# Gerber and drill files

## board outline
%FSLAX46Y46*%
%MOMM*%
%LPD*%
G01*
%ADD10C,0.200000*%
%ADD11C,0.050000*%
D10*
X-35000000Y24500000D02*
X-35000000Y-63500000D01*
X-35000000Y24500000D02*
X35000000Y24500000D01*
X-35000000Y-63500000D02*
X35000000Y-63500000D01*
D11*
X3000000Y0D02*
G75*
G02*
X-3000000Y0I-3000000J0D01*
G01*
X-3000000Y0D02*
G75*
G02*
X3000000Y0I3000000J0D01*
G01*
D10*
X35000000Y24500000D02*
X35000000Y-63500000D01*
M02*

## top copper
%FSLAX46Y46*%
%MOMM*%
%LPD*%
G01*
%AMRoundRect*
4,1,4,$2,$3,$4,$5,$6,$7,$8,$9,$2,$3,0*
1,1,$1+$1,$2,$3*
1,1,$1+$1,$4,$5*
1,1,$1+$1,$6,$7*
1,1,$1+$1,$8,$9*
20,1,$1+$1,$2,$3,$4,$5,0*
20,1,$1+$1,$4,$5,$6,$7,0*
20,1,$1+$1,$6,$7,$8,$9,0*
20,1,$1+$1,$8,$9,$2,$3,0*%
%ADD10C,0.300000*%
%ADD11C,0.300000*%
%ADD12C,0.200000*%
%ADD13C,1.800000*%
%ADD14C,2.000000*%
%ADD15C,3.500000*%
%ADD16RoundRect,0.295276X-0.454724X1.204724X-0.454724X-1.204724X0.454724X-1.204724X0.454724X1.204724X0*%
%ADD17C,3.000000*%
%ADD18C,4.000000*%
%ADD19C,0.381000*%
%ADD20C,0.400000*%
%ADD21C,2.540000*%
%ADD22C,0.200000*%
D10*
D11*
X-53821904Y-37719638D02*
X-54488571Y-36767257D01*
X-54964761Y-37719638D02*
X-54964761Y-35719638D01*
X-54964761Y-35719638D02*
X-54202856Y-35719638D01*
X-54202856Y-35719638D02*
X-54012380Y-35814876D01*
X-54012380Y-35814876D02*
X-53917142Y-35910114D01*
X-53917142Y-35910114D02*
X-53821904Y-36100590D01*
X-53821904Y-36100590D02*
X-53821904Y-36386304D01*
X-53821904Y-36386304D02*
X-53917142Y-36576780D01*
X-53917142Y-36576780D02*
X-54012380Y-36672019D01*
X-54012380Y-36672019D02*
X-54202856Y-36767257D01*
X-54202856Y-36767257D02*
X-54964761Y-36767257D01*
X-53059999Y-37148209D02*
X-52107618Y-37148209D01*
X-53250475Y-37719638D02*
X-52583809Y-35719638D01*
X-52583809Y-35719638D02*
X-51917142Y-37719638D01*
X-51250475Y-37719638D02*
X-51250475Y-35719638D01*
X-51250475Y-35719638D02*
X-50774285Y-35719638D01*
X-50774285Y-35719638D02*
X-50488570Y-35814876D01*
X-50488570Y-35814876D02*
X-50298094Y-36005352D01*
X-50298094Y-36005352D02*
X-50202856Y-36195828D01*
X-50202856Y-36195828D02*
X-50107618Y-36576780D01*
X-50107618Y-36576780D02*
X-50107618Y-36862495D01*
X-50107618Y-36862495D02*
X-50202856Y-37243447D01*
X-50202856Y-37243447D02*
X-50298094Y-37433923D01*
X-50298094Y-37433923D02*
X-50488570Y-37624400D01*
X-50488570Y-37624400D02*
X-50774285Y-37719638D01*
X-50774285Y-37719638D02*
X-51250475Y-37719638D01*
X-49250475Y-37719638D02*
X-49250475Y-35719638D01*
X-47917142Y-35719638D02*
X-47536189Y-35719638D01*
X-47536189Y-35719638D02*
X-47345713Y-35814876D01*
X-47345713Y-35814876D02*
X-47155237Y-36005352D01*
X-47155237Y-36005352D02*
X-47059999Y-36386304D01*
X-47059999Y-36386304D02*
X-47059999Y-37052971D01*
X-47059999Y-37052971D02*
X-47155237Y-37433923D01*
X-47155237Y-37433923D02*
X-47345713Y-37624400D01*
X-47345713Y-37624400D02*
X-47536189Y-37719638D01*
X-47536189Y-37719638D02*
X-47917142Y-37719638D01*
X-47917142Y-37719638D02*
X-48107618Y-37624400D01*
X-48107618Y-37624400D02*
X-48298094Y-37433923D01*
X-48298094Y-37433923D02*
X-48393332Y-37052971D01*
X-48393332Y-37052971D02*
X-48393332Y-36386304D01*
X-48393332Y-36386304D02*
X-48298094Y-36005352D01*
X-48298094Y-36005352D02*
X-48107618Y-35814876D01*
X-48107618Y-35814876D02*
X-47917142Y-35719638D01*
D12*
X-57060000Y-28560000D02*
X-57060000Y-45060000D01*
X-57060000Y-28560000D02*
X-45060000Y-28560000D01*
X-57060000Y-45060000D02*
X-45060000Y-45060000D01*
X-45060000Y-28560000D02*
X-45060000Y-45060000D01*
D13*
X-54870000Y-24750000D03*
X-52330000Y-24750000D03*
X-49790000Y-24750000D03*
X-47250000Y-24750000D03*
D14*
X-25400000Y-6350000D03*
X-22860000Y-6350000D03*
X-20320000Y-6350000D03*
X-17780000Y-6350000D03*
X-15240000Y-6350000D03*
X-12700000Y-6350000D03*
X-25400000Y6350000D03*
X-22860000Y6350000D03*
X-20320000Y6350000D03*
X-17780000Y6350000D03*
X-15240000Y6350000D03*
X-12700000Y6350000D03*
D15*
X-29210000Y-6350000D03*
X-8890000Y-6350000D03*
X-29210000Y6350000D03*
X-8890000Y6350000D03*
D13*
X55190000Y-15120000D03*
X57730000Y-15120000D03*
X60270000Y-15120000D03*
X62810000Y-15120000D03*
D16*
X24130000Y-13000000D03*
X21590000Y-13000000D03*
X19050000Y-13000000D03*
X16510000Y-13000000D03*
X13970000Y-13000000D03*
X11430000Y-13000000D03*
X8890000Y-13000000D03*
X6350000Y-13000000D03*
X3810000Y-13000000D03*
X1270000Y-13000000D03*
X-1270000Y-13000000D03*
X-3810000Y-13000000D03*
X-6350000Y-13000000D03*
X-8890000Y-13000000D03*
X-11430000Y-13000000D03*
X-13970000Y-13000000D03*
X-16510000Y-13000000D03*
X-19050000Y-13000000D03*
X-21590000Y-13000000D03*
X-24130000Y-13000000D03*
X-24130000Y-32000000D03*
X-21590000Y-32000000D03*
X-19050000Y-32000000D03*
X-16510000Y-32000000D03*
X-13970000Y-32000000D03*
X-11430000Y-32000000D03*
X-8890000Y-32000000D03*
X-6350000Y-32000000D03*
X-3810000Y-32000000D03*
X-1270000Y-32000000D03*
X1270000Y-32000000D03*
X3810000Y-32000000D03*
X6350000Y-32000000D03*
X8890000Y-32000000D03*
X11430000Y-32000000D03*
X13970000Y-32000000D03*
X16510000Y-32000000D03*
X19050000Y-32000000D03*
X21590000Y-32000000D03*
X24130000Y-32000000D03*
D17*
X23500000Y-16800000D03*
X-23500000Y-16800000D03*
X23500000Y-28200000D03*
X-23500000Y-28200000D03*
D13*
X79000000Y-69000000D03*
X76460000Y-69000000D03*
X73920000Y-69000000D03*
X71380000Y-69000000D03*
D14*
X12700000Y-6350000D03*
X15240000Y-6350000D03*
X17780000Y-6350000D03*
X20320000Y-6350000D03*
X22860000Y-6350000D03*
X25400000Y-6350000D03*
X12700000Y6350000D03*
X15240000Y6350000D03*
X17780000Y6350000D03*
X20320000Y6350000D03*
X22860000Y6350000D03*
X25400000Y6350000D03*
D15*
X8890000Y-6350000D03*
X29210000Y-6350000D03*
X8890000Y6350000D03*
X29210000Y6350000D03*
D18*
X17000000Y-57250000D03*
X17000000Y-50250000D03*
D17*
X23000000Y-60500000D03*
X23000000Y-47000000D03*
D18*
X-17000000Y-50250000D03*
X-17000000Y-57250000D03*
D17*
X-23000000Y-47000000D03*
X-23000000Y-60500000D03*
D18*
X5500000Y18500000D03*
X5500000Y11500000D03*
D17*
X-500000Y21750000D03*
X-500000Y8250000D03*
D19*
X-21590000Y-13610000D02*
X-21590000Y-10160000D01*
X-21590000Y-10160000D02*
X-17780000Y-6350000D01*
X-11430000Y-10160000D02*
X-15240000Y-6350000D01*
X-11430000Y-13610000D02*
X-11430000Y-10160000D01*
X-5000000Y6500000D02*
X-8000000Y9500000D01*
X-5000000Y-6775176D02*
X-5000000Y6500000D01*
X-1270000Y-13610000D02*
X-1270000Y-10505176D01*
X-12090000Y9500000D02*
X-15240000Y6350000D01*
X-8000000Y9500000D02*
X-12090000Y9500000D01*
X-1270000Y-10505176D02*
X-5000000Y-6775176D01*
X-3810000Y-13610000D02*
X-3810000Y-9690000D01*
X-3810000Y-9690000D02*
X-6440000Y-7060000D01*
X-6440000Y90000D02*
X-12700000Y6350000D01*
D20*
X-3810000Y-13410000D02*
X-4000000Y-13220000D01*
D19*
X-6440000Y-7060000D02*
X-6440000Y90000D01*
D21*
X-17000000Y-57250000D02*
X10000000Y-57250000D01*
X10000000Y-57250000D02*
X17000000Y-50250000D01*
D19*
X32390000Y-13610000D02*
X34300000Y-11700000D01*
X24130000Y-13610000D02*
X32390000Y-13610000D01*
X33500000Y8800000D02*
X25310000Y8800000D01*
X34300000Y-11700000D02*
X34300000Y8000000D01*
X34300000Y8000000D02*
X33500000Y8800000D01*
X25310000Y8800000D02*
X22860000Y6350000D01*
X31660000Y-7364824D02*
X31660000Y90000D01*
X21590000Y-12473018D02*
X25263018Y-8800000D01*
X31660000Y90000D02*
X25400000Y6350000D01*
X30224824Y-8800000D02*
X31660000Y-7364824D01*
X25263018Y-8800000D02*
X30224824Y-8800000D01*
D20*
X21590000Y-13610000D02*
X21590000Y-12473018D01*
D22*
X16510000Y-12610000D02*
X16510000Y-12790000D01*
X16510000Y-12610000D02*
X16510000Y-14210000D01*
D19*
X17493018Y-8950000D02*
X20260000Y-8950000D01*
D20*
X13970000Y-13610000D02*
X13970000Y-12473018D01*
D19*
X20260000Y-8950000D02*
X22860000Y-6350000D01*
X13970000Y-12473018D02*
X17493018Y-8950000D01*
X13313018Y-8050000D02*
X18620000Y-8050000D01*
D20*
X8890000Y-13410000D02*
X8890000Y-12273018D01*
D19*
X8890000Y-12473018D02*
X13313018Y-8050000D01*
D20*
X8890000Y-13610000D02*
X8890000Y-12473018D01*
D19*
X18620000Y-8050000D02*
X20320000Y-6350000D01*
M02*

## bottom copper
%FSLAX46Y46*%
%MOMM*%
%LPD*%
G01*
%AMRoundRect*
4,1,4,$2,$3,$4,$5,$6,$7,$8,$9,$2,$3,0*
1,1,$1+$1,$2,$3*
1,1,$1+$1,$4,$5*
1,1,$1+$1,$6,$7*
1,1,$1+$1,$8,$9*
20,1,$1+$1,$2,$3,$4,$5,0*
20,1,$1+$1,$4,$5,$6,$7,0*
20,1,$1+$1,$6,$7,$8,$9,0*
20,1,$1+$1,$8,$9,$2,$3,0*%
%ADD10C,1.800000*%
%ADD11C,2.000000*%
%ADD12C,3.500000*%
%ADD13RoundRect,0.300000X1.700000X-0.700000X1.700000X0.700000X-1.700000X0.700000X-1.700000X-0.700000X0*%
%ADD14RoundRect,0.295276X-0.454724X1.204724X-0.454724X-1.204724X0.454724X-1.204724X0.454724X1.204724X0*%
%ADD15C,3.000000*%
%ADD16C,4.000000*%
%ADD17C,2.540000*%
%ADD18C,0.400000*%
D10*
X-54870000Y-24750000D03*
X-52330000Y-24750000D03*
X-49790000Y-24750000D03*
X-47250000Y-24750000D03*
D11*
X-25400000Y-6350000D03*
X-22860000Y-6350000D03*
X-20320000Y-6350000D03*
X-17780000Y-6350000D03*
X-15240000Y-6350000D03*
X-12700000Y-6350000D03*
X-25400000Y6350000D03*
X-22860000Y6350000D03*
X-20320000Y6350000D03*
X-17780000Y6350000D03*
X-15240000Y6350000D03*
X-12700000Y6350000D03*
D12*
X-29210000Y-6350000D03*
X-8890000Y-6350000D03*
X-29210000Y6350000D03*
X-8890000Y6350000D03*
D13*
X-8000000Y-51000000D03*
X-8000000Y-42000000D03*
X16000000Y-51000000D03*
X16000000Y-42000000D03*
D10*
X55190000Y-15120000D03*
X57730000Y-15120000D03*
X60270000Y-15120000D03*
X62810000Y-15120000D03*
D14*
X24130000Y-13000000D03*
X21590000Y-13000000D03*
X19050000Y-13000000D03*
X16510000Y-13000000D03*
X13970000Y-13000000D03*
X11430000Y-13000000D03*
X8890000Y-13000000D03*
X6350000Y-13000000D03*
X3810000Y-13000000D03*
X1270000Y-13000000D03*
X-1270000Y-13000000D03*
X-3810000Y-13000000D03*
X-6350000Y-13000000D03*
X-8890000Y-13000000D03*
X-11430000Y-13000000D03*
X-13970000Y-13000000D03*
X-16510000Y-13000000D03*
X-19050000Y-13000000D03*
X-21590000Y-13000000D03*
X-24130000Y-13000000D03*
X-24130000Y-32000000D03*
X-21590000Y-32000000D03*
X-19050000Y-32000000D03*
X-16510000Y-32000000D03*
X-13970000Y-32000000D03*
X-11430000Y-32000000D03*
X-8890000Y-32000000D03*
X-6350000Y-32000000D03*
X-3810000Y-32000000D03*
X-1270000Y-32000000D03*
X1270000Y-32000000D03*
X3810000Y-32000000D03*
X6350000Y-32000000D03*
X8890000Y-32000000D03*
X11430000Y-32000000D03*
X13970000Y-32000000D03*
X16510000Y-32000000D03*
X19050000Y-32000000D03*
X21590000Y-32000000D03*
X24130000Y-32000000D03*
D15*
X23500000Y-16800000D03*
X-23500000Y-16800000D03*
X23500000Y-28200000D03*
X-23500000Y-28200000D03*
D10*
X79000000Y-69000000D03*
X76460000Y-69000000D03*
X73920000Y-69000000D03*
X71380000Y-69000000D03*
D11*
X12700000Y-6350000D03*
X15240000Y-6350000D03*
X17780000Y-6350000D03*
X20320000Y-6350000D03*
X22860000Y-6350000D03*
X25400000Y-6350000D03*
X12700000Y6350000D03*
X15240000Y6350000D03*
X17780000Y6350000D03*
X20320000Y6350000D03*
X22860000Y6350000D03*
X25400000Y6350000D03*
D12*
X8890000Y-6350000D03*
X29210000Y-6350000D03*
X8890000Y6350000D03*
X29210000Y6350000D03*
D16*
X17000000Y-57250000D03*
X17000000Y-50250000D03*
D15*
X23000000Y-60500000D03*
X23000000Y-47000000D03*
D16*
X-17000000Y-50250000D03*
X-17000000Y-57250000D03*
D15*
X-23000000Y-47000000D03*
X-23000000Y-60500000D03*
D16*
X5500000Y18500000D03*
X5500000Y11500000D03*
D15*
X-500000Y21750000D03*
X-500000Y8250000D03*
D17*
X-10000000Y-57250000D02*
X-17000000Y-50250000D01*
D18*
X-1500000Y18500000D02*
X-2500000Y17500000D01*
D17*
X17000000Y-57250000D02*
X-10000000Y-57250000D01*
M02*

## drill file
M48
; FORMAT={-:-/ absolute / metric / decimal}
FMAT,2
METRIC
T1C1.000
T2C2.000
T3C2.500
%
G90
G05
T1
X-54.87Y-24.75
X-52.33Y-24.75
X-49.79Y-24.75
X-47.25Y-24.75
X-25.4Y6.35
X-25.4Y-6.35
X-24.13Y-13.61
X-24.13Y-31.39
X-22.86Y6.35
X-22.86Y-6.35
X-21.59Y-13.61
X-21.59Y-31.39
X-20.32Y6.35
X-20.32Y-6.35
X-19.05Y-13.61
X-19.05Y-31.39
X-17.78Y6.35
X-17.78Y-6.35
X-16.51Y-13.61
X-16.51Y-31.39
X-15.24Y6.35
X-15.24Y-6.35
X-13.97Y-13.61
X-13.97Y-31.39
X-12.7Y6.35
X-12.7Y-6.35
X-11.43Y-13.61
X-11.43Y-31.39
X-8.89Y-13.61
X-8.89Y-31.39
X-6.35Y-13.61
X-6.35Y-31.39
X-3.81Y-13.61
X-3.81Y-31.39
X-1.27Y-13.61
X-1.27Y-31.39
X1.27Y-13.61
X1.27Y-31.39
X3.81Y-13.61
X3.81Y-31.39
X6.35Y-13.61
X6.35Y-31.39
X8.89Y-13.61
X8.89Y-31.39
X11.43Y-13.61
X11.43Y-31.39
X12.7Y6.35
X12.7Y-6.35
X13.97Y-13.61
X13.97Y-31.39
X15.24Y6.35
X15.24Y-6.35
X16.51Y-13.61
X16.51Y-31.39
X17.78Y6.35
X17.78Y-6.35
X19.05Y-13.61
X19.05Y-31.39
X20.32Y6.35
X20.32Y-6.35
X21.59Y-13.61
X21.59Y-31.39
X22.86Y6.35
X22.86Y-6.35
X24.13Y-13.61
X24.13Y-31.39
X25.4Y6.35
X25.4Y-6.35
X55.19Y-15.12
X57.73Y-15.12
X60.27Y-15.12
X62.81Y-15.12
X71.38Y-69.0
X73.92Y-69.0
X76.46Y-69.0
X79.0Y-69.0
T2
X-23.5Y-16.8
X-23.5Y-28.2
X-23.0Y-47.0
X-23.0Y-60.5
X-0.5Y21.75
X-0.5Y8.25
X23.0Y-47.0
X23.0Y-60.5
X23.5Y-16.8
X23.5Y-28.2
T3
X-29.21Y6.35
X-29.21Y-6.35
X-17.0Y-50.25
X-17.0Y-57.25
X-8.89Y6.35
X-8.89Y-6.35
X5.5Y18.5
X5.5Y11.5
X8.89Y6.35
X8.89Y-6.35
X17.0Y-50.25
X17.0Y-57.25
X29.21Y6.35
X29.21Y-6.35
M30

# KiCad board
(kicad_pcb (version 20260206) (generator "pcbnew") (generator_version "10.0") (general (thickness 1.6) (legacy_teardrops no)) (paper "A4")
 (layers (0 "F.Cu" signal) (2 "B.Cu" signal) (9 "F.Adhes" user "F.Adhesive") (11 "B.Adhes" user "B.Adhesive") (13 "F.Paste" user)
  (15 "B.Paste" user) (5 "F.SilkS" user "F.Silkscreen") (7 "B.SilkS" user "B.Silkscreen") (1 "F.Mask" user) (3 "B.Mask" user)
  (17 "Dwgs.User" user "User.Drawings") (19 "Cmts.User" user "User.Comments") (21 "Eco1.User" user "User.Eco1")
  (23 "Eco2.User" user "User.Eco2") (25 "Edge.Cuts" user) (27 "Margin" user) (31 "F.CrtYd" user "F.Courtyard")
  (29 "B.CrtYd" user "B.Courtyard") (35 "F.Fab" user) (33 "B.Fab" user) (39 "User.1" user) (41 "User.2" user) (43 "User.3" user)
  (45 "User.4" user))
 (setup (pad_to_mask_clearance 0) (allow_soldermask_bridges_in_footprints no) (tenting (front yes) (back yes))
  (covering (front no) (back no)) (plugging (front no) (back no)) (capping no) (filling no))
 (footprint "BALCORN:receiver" (layer "F.Cu") (at -51.06 36.81)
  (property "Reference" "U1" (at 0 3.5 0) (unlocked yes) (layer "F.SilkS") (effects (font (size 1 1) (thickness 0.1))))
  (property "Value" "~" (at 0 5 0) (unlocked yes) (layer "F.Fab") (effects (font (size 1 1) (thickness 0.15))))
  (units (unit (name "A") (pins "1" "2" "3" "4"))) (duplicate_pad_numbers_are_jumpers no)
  (fp_line (start -6 -8.25) (end -6 8.25) (stroke (width 0.2) (type default)) (layer "F.Cu"))
  (fp_line (start -6 -8.25) (end 6 -8.25) (stroke (width 0.2) (type default)) (layer "F.Cu"))
  (fp_line (start -6 8.25) (end 6 8.25) (stroke (width 0.2) (type default)) (layer "F.Cu"))
  (fp_line (start 6 -8.25) (end 6 8.25) (stroke (width 0.2) (type default)) (layer "F.Cu"))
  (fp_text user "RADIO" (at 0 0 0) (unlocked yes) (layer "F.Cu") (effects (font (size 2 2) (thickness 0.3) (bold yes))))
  (pad "1" thru_hole circle (at -3.81 -12.06) (size 1.8 1.8) (drill 1) (layers "*.Cu" "*.Mask") (remove_unused_layers no)
   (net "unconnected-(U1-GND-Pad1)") (thermal_bridge_angle 90))
  (pad "2" thru_hole circle (at -1.27 -12.06) (size 1.8 1.8) (drill 1) (layers "*.Cu" "*.Mask") (remove_unused_layers no)
   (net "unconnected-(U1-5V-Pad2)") (thermal_bridge_angle 90))
  (pad "3" thru_hole circle (at 1.27 -12.06) (size 1.8 1.8) (drill 1) (layers "*.Cu" "*.Mask") (remove_unused_layers no)
   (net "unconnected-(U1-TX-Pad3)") (thermal_bridge_angle 90))
  (pad "4" thru_hole circle (at 3.81 -12.06) (size 1.8 1.8) (drill 1) (layers "*.Cu" "*.Mask") (remove_unused_layers no)
   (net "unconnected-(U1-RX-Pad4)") (thermal_bridge_angle 90)))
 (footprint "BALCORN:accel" (layer "F.Cu") (at -19.05 0 90)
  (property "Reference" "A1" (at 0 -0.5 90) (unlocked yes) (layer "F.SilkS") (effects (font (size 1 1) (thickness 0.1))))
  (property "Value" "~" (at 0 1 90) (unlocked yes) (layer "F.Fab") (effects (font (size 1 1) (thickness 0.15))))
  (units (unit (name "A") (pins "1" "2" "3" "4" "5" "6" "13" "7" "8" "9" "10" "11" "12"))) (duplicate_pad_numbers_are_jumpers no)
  (pad "1" thru_hole circle (at -6.35 -6.35 90) (size 2 2) (drill 1) (layers "*.Cu" "*.Mask") (remove_unused_layers no) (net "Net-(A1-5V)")
   (thermal_bridge_angle 90))
  (pad "2" thru_hole circle (at -6.35 -3.81 90) (size 2 2) (drill 1) (layers "*.Cu" "*.Mask") (remove_unused_layers no)
   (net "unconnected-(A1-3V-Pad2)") (thermal_bridge_angle 90))
  (pad "3" thru_hole circle (at -6.35 -1.27 90) (size 2 2) (drill 1) (layers "*.Cu" "*.Mask") (remove_unused_layers no)
   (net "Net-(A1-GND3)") (thermal_bridge_angle 90))
  (pad "4" thru_hole circle (at -6.35 1.27 90) (size 2 2) (drill 1) (layers "*.Cu" "*.Mask") (remove_unused_layers no) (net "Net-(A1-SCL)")
   (thermal_bridge_angle 90))
  (pad "5" thru_hole circle (at -6.35 3.81 90) (size 2 2) (drill 1) (layers "*.Cu" "*.Mask") (remove_unused_layers no) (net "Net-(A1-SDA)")
   (thermal_bridge_angle 90))
  (pad "6" thru_hole circle (at -6.35 6.35 90) (size 2 2) (drill 1) (layers "*.Cu" "*.Mask") (remove_unused_layers no)
   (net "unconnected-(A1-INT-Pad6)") (thermal_bridge_angle 90))
  (pad "7" thru_hole circle (at 6.35 -6.35 90) (size 2 2) (drill 1) (layers "*.Cu" "*.Mask") (remove_unused_layers no)
   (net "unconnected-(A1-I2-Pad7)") (thermal_bridge_angle 90))
  (pad "8" thru_hole circle (at 6.35 -3.81 90) (size 2 2) (drill 1) (layers "*.Cu" "*.Mask") (remove_unused_layers no)
   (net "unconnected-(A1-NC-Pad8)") (thermal_bridge_angle 90))
  (pad "9" thru_hole circle (at 6.35 -1.27 90) (size 2 2) (drill 1) (layers "*.Cu" "*.Mask") (remove_unused_layers no)
   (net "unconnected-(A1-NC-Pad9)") (thermal_bridge_angle 90))
  (pad "10" thru_hole circle (at 6.35 1.27 90) (size 2 2) (drill 1) (layers "*.Cu" "*.Mask") (remove_unused_layers no)
   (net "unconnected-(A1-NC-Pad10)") (thermal_bridge_angle 90))
  (pad "11" thru_hole circle (at 6.35 3.81 90) (size 2 2) (drill 1) (layers "*.Cu" "*.Mask") (remove_unused_layers no) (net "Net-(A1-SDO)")
   (thermal_bridge_angle 90))
  (pad "12" thru_hole circle (at 6.35 6.35 90) (size 2 2) (drill 1) (layers "*.Cu" "*.Mask") (remove_unused_layers no) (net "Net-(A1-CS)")
   (thermal_bridge_angle 90))
  (pad "13" thru_hole circle (at -6.35 -10.16 90) (size 3.5 3.5) (drill 2.5) (layers "*.Cu" "*.Mask") (remove_unused_layers no)
   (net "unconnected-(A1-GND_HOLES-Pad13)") (thermal_bridge_angle 90))
  (pad "13" thru_hole circle (at -6.35 10.16 90) (size 3.5 3.5) (drill 2.5) (layers "*.Cu" "*.Mask") (remove_unused_layers no)
   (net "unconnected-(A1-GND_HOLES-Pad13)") (thermal_bridge_angle 90))
  (pad "13" thru_hole circle (at 6.35 -10.16 90) (size 3.5 3.5) (drill 2.5) (layers "*.Cu" "*.Mask") (remove_unused_layers no)
   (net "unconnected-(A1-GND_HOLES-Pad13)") (thermal_bridge_angle 90))
  (pad "13" thru_hole circle (at 6.35 10.16 90) (size 3.5 3.5) (drill 2.5) (layers "*.Cu" "*.Mask") (remove_unused_layers no)
   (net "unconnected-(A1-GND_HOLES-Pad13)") (thermal_bridge_angle 90)))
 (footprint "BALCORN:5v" (layer "F.Cu") (at 4 46.5 90)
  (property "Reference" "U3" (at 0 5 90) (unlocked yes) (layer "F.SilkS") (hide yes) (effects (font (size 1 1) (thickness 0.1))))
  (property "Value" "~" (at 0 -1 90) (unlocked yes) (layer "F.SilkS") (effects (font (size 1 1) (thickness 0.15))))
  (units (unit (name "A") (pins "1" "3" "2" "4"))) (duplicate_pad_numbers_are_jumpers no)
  (pad "1" smd roundrect (at -4.5 -12 90) (size 2 4) (layers "*.Mask" "B.Cu") (roundrect_rratio 0.15) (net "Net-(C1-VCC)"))
  (pad "2" smd roundrect (at 4.5 -12 90) (size 2 4) (layers "*.Mask" "B.Cu") (roundrect_rratio 0.15) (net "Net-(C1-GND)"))
  (pad "3" smd roundrect (at -4.5 12 90) (size 2 4) (layers "*.Mask" "B.Cu") (roundrect_rratio 0.15) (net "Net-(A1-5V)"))
  (pad "4" smd roundrect (at 4.5 12 90) (size 2 4) (layers "*.Mask" "B.Cu") (roundrect_rratio 0.15) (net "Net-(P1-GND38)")))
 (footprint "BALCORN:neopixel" (layer "F.Cu") (at 59 15.12)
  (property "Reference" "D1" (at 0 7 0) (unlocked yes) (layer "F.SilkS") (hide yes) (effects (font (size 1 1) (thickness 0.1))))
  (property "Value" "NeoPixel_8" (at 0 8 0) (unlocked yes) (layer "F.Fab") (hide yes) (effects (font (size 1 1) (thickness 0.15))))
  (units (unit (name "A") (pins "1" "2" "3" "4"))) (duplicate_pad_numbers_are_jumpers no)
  (pad "1" thru_hole circle (at -3.81 0) (size 1.8 1.8) (drill 1) (layers "*.Cu" "*.Mask") (remove_unused_layers no)
   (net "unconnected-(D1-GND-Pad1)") (thermal_bridge_angle 90))
  (pad "2" thru_hole circle (at -1.27 0) (size 1.8 1.8) (drill 1) (layers "*.Cu" "*.Mask") (remove_unused_layers no)
   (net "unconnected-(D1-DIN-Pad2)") (thermal_bridge_angle 90))
  (pad "3" thru_hole circle (at 1.27 0) (size 1.8 1.8) (drill 1) (layers "*.Cu" "*.Mask") (remove_unused_layers no)
   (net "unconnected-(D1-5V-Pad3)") (thermal_bridge_angle 90))
  (pad "4" thru_hole circle (at 3.81 0) (size 1.8 1.8) (drill 1) (layers "*.Cu" "*.Mask") (remove_unused_layers no)
   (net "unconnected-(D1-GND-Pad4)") (thermal_bridge_angle 90)))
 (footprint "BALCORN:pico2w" (layer "F.Cu") (at 0 22.5 -90)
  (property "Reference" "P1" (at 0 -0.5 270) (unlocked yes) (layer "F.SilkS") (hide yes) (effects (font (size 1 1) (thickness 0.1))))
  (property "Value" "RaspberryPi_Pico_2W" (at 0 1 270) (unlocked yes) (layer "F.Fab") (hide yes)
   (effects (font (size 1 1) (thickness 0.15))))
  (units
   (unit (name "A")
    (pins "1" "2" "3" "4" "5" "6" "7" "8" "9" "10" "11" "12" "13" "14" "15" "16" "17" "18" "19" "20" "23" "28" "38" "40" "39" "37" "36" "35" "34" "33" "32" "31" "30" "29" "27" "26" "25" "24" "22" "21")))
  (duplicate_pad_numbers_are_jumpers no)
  (pad "1" thru_hole roundrect (at -8.89 -24.13 270) (size 3 1.5) (drill 1 (offset -0.61 0)) (layers "*.Cu" "*.Mask")
   (remove_unused_layers no) (roundrect_rratio 0.1968503937) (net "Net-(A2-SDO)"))
  (pad "2" thru_hole roundrect (at -8.89 -21.59 270) (size 3 1.5) (drill 1 (offset -0.61 0)) (layers "*.Cu" "*.Mask")
   (remove_unused_layers no) (roundrect_rratio 0.1968503937) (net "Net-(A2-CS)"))
  (pad "3" thru_hole roundrect (at -8.89 -19.05 270) (size 3 1.5) (drill 1 (offset -0.61 0)) (layers "*.Cu" "*.Mask")
   (remove_unused_layers no) (roundrect_rratio 0.1968503937) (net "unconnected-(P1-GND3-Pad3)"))
  (pad "4" thru_hole roundrect (at -8.89 -16.51 270) (size 3 1.5) (drill 1 (offset -0.61 0)) (layers "*.Cu" "*.Mask")
   (remove_unused_layers no) (roundrect_rratio 0.1968503937) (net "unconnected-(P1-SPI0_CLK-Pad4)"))
  (pad "5" thru_hole roundrect (at -8.89 -13.97 270) (size 3 1.5) (drill 1 (offset -0.61 0)) (layers "*.Cu" "*.Mask")
   (remove_unused_layers no) (roundrect_rratio 0.1968503937) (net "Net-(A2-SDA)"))
  (pad "6" thru_hole roundrect (at -8.89 -11.43 270) (size 3 1.5) (drill 1 (offset -0.61 0)) (layers "*.Cu" "*.Mask")
   (remove_unused_layers no) (roundrect_rratio 0.1968503937) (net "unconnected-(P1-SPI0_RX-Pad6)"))
  (pad "7" thru_hole roundrect (at -8.89 -8.89 270) (size 3 1.5) (drill 1 (offset -0.61 0)) (layers "*.Cu" "*.Mask")
   (remove_unused_layers no) (roundrect_rratio 0.1968503937) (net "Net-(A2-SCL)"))
  (pad "8" thru_hole roundrect (at -8.89 -6.35 270) (size 3 1.5) (drill 1 (offset -0.61 0)) (layers "*.Cu" "*.Mask")
   (remove_unused_layers no) (roundrect_rratio 0.1968503937) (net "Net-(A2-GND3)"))
  (pad "9" thru_hole roundrect (at -8.89 -3.81 270) (size 3 1.5) (drill 1 (offset -0.61 0)) (layers "*.Cu" "*.Mask")
   (remove_unused_layers no) (roundrect_rratio 0.1968503937) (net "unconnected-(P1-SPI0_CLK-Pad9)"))
  (pad "10" thru_hole roundrect (at -8.89 -1.27 270) (size 3 1.5) (drill 1 (offset -0.61 0)) (layers "*.Cu" "*.Mask")
   (remove_unused_layers no) (roundrect_rratio 0.1968503937) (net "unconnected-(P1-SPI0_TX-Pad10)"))
  (pad "11" thru_hole roundrect (at -8.89 1.27 270) (size 3 1.5) (drill 1 (offset -0.61 0)) (layers "*.Cu" "*.Mask")
   (remove_unused_layers no) (roundrect_rratio 0.1968503937) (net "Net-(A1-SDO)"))
  (pad "12" thru_hole roundrect (at -8.89 3.81 270) (size 3 1.5) (drill 1 (offset -0.61 0)) (layers "*.Cu" "*.Mask")
   (remove_unused_layers no) (roundrect_rratio 0.1968503937) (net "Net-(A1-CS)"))
  (pad "13" thru_hole roundrect (at -8.89 6.35 270) (size 3 1.5) (drill 1 (offset -0.61 0)) (layers "*.Cu" "*.Mask")
   (remove_unused_layers no) (roundrect_rratio 0.1968503937) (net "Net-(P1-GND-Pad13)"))
  (pad "14" thru_hole roundrect (at -8.89 8.89 270) (size 3 1.5) (drill 1 (offset -0.61 0)) (layers "*.Cu" "*.Mask")
   (remove_unused_layers no) (roundrect_rratio 0.1968503937) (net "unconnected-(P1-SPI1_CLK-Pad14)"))
  (pad "15" thru_hole roundrect (at -8.89 11.43 270) (size 3 1.5) (drill 1 (offset -0.61 0)) (layers "*.Cu" "*.Mask")
   (remove_unused_layers no) (roundrect_rratio 0.1968503937) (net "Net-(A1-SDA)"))
  (pad "16" thru_hole roundrect (at -8.89 13.97 270) (size 3 1.5) (drill 1 (offset -0.61 0)) (layers "*.Cu" "*.Mask")
   (remove_unused_layers no) (roundrect_rratio 0.1968503937) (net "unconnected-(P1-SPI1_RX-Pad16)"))
  (pad "17" thru_hole roundrect (at -8.89 16.51 270) (size 3 1.5) (drill 1 (offset -0.61 0)) (layers "*.Cu" "*.Mask")
   (remove_unused_layers no) (roundrect_rratio 0.1968503937) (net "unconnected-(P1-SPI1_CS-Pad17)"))
  (pad "18" thru_hole roundrect (at -8.89 19.05 270) (size 3 1.5) (drill 1 (offset -0.61 0)) (layers "*.Cu" "*.Mask")
   (remove_unused_layers no) (roundrect_rratio 0.1968503937) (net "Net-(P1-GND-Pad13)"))
  (pad "19" thru_hole roundrect (at -8.89 21.59 270) (size 3 1.5) (drill 1 (offset -0.61 0)) (layers "*.Cu" "*.Mask")
   (remove_unused_layers no) (roundrect_rratio 0.1968503937) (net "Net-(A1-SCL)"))
  (pad "20" thru_hole roundrect (at -8.89 24.13 270) (size 3 1.5) (drill 1 (offset -0.61 0)) (layers "*.Cu" "*.Mask")
   (remove_unused_layers no) (roundrect_rratio 0.1968503937) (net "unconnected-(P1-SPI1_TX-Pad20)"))
  (pad "21" thru_hole roundrect (at 8.89 24.13 270) (size 3 1.5) (drill 1 (offset 0.61 0)) (layers "*.Cu" "*.Mask")
   (remove_unused_layers no) (roundrect_rratio 0.1968503937) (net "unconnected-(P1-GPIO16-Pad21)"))
  (pad "22" thru_hole roundrect (at 8.89 21.59 270) (size 3 1.5) (drill 1 (offset 0.61 0)) (layers "*.Cu" "*.Mask")
   (remove_unused_layers no) (roundrect_rratio 0.1968503937) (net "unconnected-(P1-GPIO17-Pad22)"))
  (pad "23" thru_hole roundrect (at 8.89 19.05 270) (size 3 1.5) (drill 1 (offset 0.61 0)) (layers "*.Cu" "*.Mask")
   (remove_unused_layers no) (roundrect_rratio 0.1968503937) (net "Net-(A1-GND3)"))
  (pad "24" thru_hole roundrect (at 8.89 16.51 270) (size 3 1.5) (drill 1 (offset 0.61 0)) (layers "*.Cu" "*.Mask")
   (remove_unused_layers no) (roundrect_rratio 0.1968503937) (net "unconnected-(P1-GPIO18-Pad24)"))
  (pad "25" thru_hole roundrect (at 8.89 13.97 270) (size 3 1.5) (drill 1 (offset 0.61 0)) (layers "*.Cu" "*.Mask")
   (remove_unused_layers no) (roundrect_rratio 0.1968503937) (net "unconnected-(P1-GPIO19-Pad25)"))
  (pad "26" thru_hole roundrect (at 8.89 11.43 270) (size 3 1.5) (drill 1 (offset 0.61 0)) (layers "*.Cu" "*.Mask")
   (remove_unused_layers no) (roundrect_rratio 0.1968503937) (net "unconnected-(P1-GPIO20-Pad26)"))
  (pad "27" thru_hole roundrect (at 8.89 8.89 270) (size 3 1.5) (drill 1 (offset 0.61 0)) (layers "*.Cu" "*.Mask") (remove_unused_layers no)
   (roundrect_rratio 0.1968503937) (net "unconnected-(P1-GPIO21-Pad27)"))
  (pad "28" thru_hole roundrect (at 8.89 6.35 270) (size 3 1.5) (drill 1 (offset 0.61 0)) (layers "*.Cu" "*.Mask") (remove_unused_layers no)
   (roundrect_rratio 0.1968503937) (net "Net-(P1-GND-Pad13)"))
  (pad "29" thru_hole roundrect (at 8.89 3.81 270) (size 3 1.5) (drill 1 (offset 0.61 0)) (layers "*.Cu" "*.Mask") (remove_unused_layers no)
   (roundrect_rratio 0.1968503937) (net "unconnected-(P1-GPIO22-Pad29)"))
  (pad "30" thru_hole roundrect (at 8.89 1.27 270) (size 3 1.5) (drill 1 (offset 0.61 0)) (layers "*.Cu" "*.Mask") (remove_unused_layers no)
   (roundrect_rratio 0.1968503937) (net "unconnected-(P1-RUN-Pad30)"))
  (pad "31" thru_hole roundrect (at 8.89 -1.27 270) (size 3 1.5) (drill 1 (offset 0.61 0)) (layers "*.Cu" "*.Mask")
   (remove_unused_layers no) (roundrect_rratio 0.1968503937) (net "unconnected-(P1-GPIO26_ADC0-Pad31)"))
  (pad "32" thru_hole roundrect (at 8.89 -3.81 270) (size 3 1.5) (drill 1 (offset 0.61 0)) (layers "*.Cu" "*.Mask")
   (remove_unused_layers no) (roundrect_rratio 0.1968503937) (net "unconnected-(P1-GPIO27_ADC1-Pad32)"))
  (pad "33" thru_hole roundrect (at 8.89 -6.35 270) (size 3 1.5) (drill 1 (offset 0.61 0)) (layers "*.Cu" "*.Mask")
   (remove_unused_layers no) (roundrect_rratio 0.1968503937) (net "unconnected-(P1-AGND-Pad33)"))
  (pad "34" thru_hole roundrect (at 8.89 -8.89 270) (size 3 1.5) (drill 1 (offset 0.61 0)) (layers "*.Cu" "*.Mask")
   (remove_unused_layers no) (roundrect_rratio 0.1968503937) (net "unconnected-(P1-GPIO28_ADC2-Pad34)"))
  (pad "35" thru_hole roundrect (at 8.89 -11.43 270) (size 3 1.5) (drill 1 (offset 0.61 0)) (layers "*.Cu" "*.Mask")
   (remove_unused_layers no) (roundrect_rratio 0.1968503937) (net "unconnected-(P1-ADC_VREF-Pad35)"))
  (pad "36" thru_hole roundrect (at 8.89 -13.97 270) (size 3 1.5) (drill 1 (offset 0.61 0)) (layers "*.Cu" "*.Mask")
   (remove_unused_layers no) (roundrect_rratio 0.1968503937) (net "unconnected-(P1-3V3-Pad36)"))
  (pad "37" thru_hole roundrect (at 8.89 -16.51 270) (size 3 1.5) (drill 1 (offset 0.61 0)) (layers "*.Cu" "*.Mask")
   (remove_unused_layers no) (roundrect_rratio 0.1968503937) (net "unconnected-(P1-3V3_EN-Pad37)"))
  (pad "38" thru_hole roundrect (at 8.89 -19.05 270) (size 3 1.5) (drill 1 (offset 0.61 0)) (layers "*.Cu" "*.Mask")
   (remove_unused_layers no) (roundrect_rratio 0.1968503937) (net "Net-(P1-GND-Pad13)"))
  (pad "39" thru_hole roundrect (at 8.89 -21.59 270) (size 3 1.5) (drill 1 (offset 0.61 0)) (layers "*.Cu" "*.Mask")
   (remove_unused_layers no) (roundrect_rratio 0.1968503937) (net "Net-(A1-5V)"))
  (pad "40" thru_hole roundrect (at 8.89 -24.13 270) (size 3 1.5) (drill 1 (offset 0.61 0)) (layers "*.Cu" "*.Mask")
   (remove_unused_layers no) (roundrect_rratio 0.1968503937) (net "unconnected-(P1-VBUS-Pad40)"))
  (pad "41" thru_hole circle (at -5.7 -23.5 270) (size 3 3) (drill 2) (layers "*.Cu" "*.Mask") (remove_unused_layers no)
   (thermal_bridge_angle 90))
  (pad "41" thru_hole circle (at -5.7 23.5 270) (size 3 3) (drill 2) (layers "*.Cu" "*.Mask") (remove_unused_layers no)
   (thermal_bridge_angle 90))
  (pad "41" thru_hole circle (at 5.7 -23.5 270) (size 3 3) (drill 2) (layers "*.Cu" "*.Mask") (remove_unused_layers no)
   (thermal_bridge_angle 90))
  (pad "41" thru_hole circle (at 5.7 23.5 270) (size 3 3) (drill 2) (layers "*.Cu" "*.Mask") (remove_unused_layers no)
   (thermal_bridge_angle 90)))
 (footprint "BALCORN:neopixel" (layer "F.Cu") (at 75.19 69 180)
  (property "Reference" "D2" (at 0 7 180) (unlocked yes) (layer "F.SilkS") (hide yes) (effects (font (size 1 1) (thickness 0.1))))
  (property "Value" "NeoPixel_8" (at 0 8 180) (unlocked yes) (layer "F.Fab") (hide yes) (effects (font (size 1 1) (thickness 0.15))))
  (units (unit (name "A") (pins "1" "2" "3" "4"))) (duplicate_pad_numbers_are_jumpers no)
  (pad "1" thru_hole circle (at -3.81 0 180) (size 1.8 1.8) (drill 1) (layers "*.Cu" "*.Mask") (remove_unused_layers no)
   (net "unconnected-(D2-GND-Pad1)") (thermal_bridge_angle 90))
  (pad "2" thru_hole circle (at -1.27 0 180) (size 1.8 1.8) (drill 1) (layers "*.Cu" "*.Mask") (remove_unused_layers no)
   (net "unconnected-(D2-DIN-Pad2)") (thermal_bridge_angle 90))
  (pad "3" thru_hole circle (at 1.27 0 180) (size 1.8 1.8) (drill 1) (layers "*.Cu" "*.Mask") (remove_unused_layers no)
   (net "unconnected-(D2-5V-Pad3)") (thermal_bridge_angle 90))
  (pad "4" thru_hole circle (at 3.81 0 180) (size 1.8 1.8) (drill 1) (layers "*.Cu" "*.Mask") (remove_unused_layers no)
   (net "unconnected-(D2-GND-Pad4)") (thermal_bridge_angle 90)))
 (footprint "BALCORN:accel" (layer "F.Cu") (at 19.05 0 90)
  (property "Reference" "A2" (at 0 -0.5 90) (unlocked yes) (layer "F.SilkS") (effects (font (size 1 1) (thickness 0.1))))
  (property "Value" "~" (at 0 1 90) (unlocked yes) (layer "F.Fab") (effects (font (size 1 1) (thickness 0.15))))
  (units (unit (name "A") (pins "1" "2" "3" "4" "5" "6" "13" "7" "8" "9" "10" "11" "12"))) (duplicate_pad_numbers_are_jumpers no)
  (pad "1" thru_hole circle (at -6.35 -6.35 90) (size 2 2) (drill 1) (layers "*.Cu" "*.Mask") (remove_unused_layers no)
   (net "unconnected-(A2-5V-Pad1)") (thermal_bridge_angle 90))
  (pad "2" thru_hole circle (at -6.35 -3.81 90) (size 2 2) (drill 1) (layers "*.Cu" "*.Mask") (remove_unused_layers no)
   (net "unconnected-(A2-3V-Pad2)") (thermal_bridge_angle 90))
  (pad "3" thru_hole circle (at -6.35 -1.27 90) (size 2 2) (drill 1) (layers "*.Cu" "*.Mask") (remove_unused_layers no)
   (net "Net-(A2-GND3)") (thermal_bridge_angle 90))
  (pad "4" thru_hole circle (at -6.35 1.27 90) (size 2 2) (drill 1) (layers "*.Cu" "*.Mask") (remove_unused_layers no) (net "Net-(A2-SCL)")
   (thermal_bridge_angle 90))
  (pad "5" thru_hole circle (at -6.35 3.81 90) (size 2 2) (drill 1) (layers "*.Cu" "*.Mask") (remove_unused_layers no) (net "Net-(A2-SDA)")
   (thermal_bridge_angle 90))
  (pad "6" thru_hole circle (at -6.35 6.35 90) (size 2 2) (drill 1) (layers "*.Cu" "*.Mask") (remove_unused_layers no)
   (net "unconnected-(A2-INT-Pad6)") (thermal_bridge_angle 90))
  (pad "7" thru_hole circle (at 6.35 -6.35 90) (size 2 2) (drill 1) (layers "*.Cu" "*.Mask") (remove_unused_layers no)
   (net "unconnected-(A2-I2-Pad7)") (thermal_bridge_angle 90))
  (pad "8" thru_hole circle (at 6.35 -3.81 90) (size 2 2) (drill 1) (layers "*.Cu" "*.Mask") (remove_unused_layers no)
   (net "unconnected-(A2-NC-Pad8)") (thermal_bridge_angle 90))
  (pad "9" thru_hole circle (at 6.35 -1.27 90) (size 2 2) (drill 1) (layers "*.Cu" "*.Mask") (remove_unused_layers no)
   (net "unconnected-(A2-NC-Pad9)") (thermal_bridge_angle 90))
  (pad "10" thru_hole circle (at 6.35 1.27 90) (size 2 2) (drill 1) (layers "*.Cu" "*.Mask") (remove_unused_layers no)
   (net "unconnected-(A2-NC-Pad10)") (thermal_bridge_angle 90))
  (pad "11" thru_hole circle (at 6.35 3.81 90) (size 2 2) (drill 1) (layers "*.Cu" "*.Mask") (remove_unused_layers no) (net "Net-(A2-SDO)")
   (thermal_bridge_angle 90))
  (pad "12" thru_hole circle (at 6.35 6.35 90) (size 2 2) (drill 1) (layers "*.Cu" "*.Mask") (remove_unused_layers no) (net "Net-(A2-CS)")
   (thermal_bridge_angle 90))
  (pad "13" thru_hole circle (at -6.35 -10.16 90) (size 3.5 3.5) (drill 2.5) (layers "*.Cu" "*.Mask") (remove_unused_layers no)
   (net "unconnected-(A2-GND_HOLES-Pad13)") (thermal_bridge_angle 90))
  (pad "13" thru_hole circle (at -6.35 10.16 90) (size 3.5 3.5) (drill 2.5) (layers "*.Cu" "*.Mask") (remove_unused_layers no)
   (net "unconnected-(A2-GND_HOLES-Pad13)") (thermal_bridge_angle 90))
  (pad "13" thru_hole circle (at 6.35 -10.16 90) (size 3.5 3.5) (drill 2.5) (layers "*.Cu" "*.Mask") (remove_unused_layers no)
   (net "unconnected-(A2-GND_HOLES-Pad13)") (thermal_bridge_angle 90))
  (pad "13" thru_hole circle (at 6.35 10.16 90) (size 3.5 3.5) (drill 2.5) (layers "*.Cu" "*.Mask") (remove_unused_layers no)
   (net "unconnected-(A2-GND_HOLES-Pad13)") (thermal_bridge_angle 90)))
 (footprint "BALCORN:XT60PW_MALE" (layer "B.Cu") (at 24.175 53.75 90)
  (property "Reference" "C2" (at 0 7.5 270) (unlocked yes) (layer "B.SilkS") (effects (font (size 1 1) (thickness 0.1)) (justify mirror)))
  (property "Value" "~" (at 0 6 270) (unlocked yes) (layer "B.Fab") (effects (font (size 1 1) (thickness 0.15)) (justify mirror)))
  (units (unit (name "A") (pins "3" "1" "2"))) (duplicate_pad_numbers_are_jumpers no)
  (pad "1" thru_hole circle (at -3.5 -7.175 90) (size 4 4) (drill 2.5) (layers "*.Cu" "*.Mask") (remove_unused_layers no)
   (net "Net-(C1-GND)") (thermal_bridge_angle 90))
  (pad "2" thru_hole circle (at 3.5 -7.175 90) (size 4 4) (drill 2.5) (layers "*.Cu" "*.Mask") (remove_unused_layers no)
   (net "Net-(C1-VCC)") (thermal_bridge_angle 90))
  (pad "3" thru_hole circle (at -6.75 -1.175 90) (size 3 3) (drill 2) (layers "*.Cu" "*.Mask") (remove_unused_layers no)
   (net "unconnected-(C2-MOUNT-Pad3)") (thermal_bridge_angle 90))
  (pad "4" thru_hole circle (at 6.75 -1.175 90) (size 3 3) (drill 2) (layers "*.Cu" "*.Mask") (remove_unused_layers no)
   (thermal_bridge_angle 90)))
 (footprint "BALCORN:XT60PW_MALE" (layer "B.Cu") (at -24.175 53.75 -90)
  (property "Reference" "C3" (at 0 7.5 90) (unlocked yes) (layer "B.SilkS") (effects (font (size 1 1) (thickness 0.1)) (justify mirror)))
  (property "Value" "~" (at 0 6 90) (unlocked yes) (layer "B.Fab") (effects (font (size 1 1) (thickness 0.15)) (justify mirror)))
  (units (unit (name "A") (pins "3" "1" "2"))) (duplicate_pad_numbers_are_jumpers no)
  (pad "1" thru_hole circle (at -3.5 -7.175 270) (size 4 4) (drill 2.5) (layers "*.Cu" "*.Mask") (remove_unused_layers no)
   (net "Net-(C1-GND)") (thermal_bridge_angle 90))
  (pad "2" thru_hole circle (at 3.5 -7.175 270) (size 4 4) (drill 2.5) (layers "*.Cu" "*.Mask") (remove_unused_layers no)
   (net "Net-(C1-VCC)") (thermal_bridge_angle 90))
  (pad "3" thru_hole circle (at -6.75 -1.175 270) (size 3 3) (drill 2) (layers "*.Cu" "*.Mask") (remove_unused_layers no)
   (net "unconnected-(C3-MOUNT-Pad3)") (thermal_bridge_angle 90))
  (pad "4" thru_hole circle (at 6.75 -1.175 270) (size 3 3) (drill 2) (layers "*.Cu" "*.Mask") (remove_unused_layers no)
   (thermal_bridge_angle 90)))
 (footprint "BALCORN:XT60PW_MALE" (layer "B.Cu") (at -1.675 -15 -90)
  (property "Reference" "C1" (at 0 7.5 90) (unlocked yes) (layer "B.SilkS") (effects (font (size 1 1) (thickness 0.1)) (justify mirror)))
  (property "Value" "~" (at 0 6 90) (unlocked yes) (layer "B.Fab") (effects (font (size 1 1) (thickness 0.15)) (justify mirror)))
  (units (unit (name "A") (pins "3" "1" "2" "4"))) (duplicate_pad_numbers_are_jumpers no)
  (pad "1" thru_hole circle (at -3.5 -7.175 270) (size 4 4) (drill 2.5) (layers "*.Cu" "*.Mask") (remove_unused_layers no)
   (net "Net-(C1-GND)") (thermal_bridge_angle 90))
  (pad "2" thru_hole circle (at 3.5 -7.175 270) (size 4 4) (drill 2.5) (layers "*.Cu" "*.Mask") (remove_unused_layers no)
   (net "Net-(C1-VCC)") (thermal_bridge_angle 90))
  (pad "3" thru_hole circle (at -6.75 -1.175 270) (size 3 3) (drill 2) (layers "*.Cu" "*.Mask") (remove_unused_layers no)
   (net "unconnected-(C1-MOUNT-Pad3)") (thermal_bridge_angle 90))
  (pad "4" thru_hole circle (at 6.75 -1.175 270) (size 3 3) (drill 2) (layers "*.Cu" "*.Mask") (remove_unused_layers no)
   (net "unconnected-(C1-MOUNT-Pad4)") (thermal_bridge_angle 90)))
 (gr_line (start -35 -24.5) (end -35 63.5) (stroke (width 0.2) (type default)) (layer "Edge.Cuts"))
 (gr_line (start -35 -24.5) (end 35 -24.5) (stroke (width 0.2) (type default)) (layer "Edge.Cuts"))
 (gr_line (start -35 63.5) (end 35 63.5) (stroke (width 0.2) (type default)) (layer "Edge.Cuts"))
 (gr_circle (center 0 0) (end 3 0) (stroke (width 0.05) (type default)) (fill no) (layer "Edge.Cuts"))
 (gr_line (start 35 -24.5) (end 35 63.5) (stroke (width 0.2) (type default)) (layer "Edge.Cuts"))
 (segment (start -21.59 13.61) (end -21.59 10.16) (width 0.381) (layer "F.Cu") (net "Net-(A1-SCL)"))
 (segment (start -21.59 10.16) (end -17.78 6.35) (width 0.381) (layer "F.Cu") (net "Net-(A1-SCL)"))
 (segment (start -11.43 10.16) (end -15.24 6.35) (width 0.381) (layer "F.Cu") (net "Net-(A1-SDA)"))
 (segment (start -11.43 13.61) (end -11.43 10.16) (width 0.381) (layer "F.Cu") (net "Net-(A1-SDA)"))
 (segment (start -5 -6.5) (end -8 -9.5) (width 0.381) (layer "F.Cu") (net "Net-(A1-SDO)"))
 (segment (start -5 6.775176) (end -5 -6.5) (width 0.381) (layer "F.Cu") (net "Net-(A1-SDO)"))
 (segment (start -1.27 13.61) (end -1.27 10.505176) (width 0.381) (layer "F.Cu") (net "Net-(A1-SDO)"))
 (segment (start -12.09 -9.5) (end -15.24 -6.35) (width 0.381) (layer "F.Cu") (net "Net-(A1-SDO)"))
 (segment (start -8 -9.5) (end -12.09 -9.5) (width 0.381) (layer "F.Cu") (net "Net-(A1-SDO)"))
 (segment (start -1.27 10.505176) (end -5 6.775176) (width 0.381) (layer "F.Cu") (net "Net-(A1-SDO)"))
 (segment (start -3.81 13.61) (end -3.81 9.69) (width 0.381) (layer "F.Cu") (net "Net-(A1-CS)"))
 (segment (start -3.81 9.69) (end -6.44 7.06) (width 0.381) (layer "F.Cu") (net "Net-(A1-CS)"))
 (segment (start -6.44 -0.09) (end -12.7 -6.35) (width 0.381) (layer "F.Cu") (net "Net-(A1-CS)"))
 (segment (start -3.81 13.41) (end -4 13.22) (width 0.4) (layer "F.Cu") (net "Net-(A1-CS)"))
 (segment (start -6.44 7.06) (end -6.44 -0.09) (width 0.381) (layer "F.Cu") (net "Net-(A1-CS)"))
 (segment (start -17 57.25) (end 10 57.25) (width 2.54) (layer "F.Cu") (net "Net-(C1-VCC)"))
 (segment (start 10 57.25) (end 17 50.25) (width 2.54) (layer "F.Cu") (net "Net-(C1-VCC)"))
 (segment (start -10 57.25) (end -17 50.25) (width 2.54) (layer "B.Cu") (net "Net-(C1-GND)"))
 (segment (start -1.5 -18.5) (end -2.5 -17.5) (width 0.4) (layer "B.Cu") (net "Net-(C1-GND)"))
 (segment (start 17 57.25) (end -10 57.25) (width 2.54) (layer "B.Cu") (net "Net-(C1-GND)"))
 (segment (start 32.39 13.61) (end 34.3 11.7) (width 0.381) (layer "F.Cu") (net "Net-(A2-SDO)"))
 (segment (start 24.13 13.61) (end 32.39 13.61) (width 0.381) (layer "F.Cu") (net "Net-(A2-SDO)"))
 (segment (start 33.5 -8.8) (end 25.31 -8.8) (width 0.381) (layer "F.Cu") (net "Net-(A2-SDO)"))
 (segment (start 34.3 11.7) (end 34.3 -8) (width 0.381) (layer "F.Cu") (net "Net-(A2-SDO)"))
 (segment (start 34.3 -8) (end 33.5 -8.8) (width 0.381) (layer "F.Cu") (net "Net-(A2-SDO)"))
 (segment (start 25.31 -8.8) (end 22.86 -6.35) (width 0.381) (layer "F.Cu") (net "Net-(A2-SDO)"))
 (segment (start 31.66 7.364824) (end 31.66 -0.09) (width 0.381) (layer "F.Cu") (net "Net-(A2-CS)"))
 (segment (start 21.59 12.473018) (end 25.263018 8.8) (width 0.381) (layer "F.Cu") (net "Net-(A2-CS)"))
 (segment (start 31.66 -0.09) (end 25.4 -6.35) (width 0.381) (layer "F.Cu") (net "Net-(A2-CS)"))
 (segment (start 30.224824 8.8) (end 31.66 7.364824) (width 0.381) (layer "F.Cu") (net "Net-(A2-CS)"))
 (segment (start 25.263018 8.8) (end 30.224824 8.8) (width 0.381) (layer "F.Cu") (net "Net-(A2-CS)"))
 (segment (start 21.59 13.61) (end 21.59 12.473018) (width 0.4) (layer "F.Cu") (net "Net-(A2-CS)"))
 (segment (start 16.51 12.61) (end 16.51 12.79) (width 0.2) (layer "F.Cu") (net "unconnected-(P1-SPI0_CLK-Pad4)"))
 (segment (start 16.51 12.61) (end 16.51 14.21) (width 0.2) (layer "F.Cu") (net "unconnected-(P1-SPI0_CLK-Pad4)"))
 (segment (start 17.493018 8.95) (end 20.26 8.95) (width 0.381) (layer "F.Cu") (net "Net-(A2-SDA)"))
 (segment (start 13.97 13.61) (end 13.97 12.473018) (width 0.4) (layer "F.Cu") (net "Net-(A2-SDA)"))
 (segment (start 20.26 8.95) (end 22.86 6.35) (width 0.381) (layer "F.Cu") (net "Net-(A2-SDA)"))
 (segment (start 13.97 12.473018) (end 17.493018 8.95) (width 0.381) (layer "F.Cu") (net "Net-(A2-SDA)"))
 (segment (start 13.313018 8.05) (end 18.62 8.05) (width 0.381) (layer "F.Cu") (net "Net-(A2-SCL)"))
 (segment (start 8.89 13.41) (end 8.89 12.273018) (width 0.4) (layer "F.Cu") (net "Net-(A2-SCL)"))
 (segment (start 8.89 12.473018) (end 13.313018 8.05) (width 0.381) (layer "F.Cu") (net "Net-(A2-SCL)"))
 (segment (start 8.89 13.61) (end 8.89 12.473018) (width 0.4) (layer "F.Cu") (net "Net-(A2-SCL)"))
 (segment (start 18.62 8.05) (end 20.32 6.35) (width 0.381) (layer "F.Cu") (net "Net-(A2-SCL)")))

